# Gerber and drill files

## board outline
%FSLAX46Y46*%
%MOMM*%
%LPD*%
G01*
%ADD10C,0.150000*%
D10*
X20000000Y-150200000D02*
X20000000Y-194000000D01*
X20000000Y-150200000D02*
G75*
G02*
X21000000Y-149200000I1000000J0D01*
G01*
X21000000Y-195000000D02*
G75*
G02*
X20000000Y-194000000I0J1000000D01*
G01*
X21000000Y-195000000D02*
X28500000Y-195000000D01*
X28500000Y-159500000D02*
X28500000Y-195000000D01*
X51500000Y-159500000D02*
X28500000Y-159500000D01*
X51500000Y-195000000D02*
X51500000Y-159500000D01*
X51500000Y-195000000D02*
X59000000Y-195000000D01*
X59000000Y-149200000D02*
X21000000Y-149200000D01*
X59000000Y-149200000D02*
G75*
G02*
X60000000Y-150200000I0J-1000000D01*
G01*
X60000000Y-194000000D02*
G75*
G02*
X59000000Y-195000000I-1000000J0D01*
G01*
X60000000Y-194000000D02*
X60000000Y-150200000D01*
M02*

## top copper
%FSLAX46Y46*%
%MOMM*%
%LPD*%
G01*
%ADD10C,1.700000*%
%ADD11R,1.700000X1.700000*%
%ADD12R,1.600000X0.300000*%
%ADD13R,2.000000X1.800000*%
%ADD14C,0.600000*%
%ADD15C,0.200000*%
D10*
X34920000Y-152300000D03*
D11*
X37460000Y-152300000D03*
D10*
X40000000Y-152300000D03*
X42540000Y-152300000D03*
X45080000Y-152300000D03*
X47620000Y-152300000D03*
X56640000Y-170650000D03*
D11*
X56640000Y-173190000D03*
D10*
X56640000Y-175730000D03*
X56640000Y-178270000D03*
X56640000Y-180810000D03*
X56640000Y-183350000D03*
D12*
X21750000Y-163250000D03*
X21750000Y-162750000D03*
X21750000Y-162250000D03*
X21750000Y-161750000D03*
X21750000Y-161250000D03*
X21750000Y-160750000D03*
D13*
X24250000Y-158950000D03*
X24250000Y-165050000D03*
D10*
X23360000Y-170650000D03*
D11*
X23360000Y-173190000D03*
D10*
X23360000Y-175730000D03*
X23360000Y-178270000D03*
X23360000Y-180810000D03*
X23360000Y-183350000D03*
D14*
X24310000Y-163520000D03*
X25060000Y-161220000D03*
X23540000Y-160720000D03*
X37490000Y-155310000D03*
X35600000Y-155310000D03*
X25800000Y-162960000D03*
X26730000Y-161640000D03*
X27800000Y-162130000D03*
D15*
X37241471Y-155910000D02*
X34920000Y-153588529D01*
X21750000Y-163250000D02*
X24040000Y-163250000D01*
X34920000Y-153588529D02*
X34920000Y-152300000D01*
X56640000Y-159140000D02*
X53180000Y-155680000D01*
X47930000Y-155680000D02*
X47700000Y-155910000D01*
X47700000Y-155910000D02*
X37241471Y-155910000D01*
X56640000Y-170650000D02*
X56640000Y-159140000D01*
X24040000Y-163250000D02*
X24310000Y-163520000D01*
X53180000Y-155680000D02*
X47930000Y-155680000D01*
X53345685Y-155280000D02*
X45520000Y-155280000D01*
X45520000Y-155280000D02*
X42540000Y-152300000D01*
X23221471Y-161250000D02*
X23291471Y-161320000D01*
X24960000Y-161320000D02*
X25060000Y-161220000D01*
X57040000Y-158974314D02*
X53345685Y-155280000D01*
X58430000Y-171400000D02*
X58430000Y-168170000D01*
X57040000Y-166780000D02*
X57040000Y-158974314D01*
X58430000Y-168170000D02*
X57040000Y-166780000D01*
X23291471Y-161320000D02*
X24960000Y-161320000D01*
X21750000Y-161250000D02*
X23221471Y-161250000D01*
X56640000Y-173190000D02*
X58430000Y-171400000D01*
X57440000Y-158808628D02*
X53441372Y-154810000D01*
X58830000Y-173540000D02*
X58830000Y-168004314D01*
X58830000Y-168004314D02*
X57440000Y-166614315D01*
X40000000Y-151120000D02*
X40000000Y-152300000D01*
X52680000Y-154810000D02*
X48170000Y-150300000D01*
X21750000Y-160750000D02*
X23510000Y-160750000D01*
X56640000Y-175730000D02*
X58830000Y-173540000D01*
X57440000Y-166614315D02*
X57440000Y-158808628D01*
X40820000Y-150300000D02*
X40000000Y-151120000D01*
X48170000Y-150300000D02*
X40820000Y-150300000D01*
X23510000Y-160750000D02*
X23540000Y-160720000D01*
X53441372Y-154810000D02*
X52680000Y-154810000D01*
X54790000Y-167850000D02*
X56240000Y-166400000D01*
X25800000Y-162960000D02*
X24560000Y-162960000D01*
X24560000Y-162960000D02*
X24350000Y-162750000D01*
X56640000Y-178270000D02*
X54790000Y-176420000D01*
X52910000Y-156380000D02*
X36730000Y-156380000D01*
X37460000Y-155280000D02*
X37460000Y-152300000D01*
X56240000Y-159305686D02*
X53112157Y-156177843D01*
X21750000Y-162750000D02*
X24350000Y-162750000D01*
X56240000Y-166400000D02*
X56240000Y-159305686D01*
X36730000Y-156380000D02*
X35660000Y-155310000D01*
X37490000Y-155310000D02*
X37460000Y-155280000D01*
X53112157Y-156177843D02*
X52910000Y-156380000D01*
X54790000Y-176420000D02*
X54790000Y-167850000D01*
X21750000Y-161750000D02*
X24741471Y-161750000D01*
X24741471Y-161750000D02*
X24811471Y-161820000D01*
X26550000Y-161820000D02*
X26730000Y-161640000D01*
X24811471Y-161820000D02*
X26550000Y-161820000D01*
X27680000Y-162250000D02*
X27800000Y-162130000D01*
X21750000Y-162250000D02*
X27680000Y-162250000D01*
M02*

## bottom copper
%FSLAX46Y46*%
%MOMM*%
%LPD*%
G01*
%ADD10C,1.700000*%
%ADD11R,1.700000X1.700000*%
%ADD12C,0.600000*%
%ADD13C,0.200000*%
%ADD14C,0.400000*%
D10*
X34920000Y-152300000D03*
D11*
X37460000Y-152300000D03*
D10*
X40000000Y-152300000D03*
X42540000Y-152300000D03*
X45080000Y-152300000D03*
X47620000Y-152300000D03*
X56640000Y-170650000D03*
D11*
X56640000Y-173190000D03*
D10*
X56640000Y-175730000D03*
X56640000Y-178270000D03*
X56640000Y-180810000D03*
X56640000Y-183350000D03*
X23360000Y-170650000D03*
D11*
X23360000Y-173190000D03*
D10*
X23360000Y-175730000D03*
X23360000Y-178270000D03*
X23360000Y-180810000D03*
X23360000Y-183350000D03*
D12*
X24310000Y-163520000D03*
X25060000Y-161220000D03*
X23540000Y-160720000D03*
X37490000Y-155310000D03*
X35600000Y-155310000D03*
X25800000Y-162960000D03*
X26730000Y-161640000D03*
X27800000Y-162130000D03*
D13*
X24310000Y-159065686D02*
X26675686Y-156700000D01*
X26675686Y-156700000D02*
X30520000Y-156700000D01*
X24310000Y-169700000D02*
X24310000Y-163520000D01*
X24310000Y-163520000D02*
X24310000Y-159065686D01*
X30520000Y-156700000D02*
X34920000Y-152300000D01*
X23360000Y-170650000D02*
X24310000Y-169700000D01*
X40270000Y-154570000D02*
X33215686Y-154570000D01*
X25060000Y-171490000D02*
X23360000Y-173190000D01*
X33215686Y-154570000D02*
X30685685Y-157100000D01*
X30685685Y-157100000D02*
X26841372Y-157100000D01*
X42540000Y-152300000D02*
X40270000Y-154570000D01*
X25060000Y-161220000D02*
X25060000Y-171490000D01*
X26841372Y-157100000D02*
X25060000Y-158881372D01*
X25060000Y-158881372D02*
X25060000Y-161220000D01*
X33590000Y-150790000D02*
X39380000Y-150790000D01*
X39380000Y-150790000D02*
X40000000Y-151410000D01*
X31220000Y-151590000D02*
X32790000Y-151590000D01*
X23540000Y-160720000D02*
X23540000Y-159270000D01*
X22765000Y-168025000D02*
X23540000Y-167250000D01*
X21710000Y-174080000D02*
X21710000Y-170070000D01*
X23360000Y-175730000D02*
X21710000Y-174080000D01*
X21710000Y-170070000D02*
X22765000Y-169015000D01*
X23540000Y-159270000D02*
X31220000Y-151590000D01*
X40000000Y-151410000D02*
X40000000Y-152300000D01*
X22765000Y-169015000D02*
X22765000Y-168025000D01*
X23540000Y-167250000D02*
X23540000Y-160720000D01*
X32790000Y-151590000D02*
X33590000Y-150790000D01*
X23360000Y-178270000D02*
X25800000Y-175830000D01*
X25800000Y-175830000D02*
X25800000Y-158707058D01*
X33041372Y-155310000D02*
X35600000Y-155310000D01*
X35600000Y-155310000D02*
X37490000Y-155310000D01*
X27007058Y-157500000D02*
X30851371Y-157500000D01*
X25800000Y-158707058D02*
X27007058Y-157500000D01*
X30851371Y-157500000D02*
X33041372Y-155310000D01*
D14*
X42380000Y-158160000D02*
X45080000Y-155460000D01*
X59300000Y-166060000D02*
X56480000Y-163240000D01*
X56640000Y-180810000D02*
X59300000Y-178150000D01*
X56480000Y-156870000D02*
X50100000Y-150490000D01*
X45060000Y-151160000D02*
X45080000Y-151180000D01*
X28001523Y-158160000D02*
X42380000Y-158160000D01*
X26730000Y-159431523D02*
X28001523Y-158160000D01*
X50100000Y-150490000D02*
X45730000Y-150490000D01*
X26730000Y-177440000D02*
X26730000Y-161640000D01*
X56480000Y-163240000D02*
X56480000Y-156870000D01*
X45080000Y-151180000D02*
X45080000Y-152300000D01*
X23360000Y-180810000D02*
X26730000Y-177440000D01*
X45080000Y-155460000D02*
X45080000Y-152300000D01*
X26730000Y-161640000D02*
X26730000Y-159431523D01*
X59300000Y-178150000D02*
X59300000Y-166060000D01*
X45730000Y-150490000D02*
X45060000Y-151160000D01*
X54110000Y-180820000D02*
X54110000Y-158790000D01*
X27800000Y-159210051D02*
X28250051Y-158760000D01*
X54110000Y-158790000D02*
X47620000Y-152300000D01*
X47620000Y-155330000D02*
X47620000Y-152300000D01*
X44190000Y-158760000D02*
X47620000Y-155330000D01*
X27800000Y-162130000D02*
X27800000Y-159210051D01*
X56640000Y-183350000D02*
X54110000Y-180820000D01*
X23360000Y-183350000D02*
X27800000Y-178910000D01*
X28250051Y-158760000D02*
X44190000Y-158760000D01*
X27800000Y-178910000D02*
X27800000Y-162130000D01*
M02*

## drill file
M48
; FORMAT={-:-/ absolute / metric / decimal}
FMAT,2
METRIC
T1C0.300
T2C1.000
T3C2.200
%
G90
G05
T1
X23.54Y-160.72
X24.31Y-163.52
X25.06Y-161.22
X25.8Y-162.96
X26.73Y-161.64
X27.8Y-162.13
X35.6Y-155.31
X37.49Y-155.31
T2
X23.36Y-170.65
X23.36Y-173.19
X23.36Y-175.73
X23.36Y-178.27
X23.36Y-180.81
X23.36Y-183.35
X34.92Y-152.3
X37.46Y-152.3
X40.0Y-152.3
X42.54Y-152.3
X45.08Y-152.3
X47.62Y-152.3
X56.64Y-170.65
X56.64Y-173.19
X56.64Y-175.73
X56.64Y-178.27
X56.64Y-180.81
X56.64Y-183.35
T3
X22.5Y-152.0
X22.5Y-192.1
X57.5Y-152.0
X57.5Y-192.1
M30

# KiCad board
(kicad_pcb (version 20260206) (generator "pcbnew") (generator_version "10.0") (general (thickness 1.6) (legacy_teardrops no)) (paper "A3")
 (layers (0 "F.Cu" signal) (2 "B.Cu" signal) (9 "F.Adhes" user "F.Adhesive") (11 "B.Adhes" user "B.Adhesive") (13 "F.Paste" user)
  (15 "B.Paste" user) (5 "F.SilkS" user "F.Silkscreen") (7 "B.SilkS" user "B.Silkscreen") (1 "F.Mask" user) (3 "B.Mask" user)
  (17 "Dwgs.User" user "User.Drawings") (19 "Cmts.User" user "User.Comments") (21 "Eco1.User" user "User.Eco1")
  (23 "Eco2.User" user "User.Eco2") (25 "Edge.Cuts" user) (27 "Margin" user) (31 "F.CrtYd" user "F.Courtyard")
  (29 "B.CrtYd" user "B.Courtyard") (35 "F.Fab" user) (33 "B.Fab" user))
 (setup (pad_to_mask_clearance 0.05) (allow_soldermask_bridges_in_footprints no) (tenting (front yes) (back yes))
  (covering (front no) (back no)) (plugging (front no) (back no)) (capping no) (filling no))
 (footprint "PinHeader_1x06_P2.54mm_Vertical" (layer "F.Cu") (at 41.27 152.3 90)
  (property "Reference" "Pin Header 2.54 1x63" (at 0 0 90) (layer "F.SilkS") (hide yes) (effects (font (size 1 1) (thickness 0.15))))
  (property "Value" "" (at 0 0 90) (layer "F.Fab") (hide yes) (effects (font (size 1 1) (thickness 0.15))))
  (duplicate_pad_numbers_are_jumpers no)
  (pad "1" thru_hole circle (at 0 -6.35 90) (size 1.7 1.7) (drill 1) (layers "*.Cu" "*.Mask") (remove_unused_layers no) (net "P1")
   (thermal_bridge_angle 90))
  (pad "2" thru_hole rect (at 0 -3.81 90) (size 1.7 1.7) (drill 1) (layers "*.Cu" "*.Mask") (remove_unused_layers no) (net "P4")
   (thermal_bridge_angle 45))
  (pad "3" thru_hole circle (at 0 -1.27 90) (size 1.7 1.7) (drill 1) (layers "*.Cu" "*.Mask") (remove_unused_layers no) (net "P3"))
  (pad "4" thru_hole circle (at 0 1.27 90) (size 1.7 1.7) (drill 1) (layers "*.Cu" "*.Mask") (remove_unused_layers no) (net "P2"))
  (pad "5" thru_hole circle (at 0 3.81 90) (size 1.7 1.7) (drill 1) (layers "*.Cu" "*.Mask") (remove_unused_layers no) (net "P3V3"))
  (pad "6" thru_hole circle (at 0 6.35 90) (size 1.7 1.7) (drill 1) (layers "*.Cu" "*.Mask") (remove_unused_layers no) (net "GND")))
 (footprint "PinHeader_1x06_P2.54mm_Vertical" (layer "F.Cu") (at 56.64 177)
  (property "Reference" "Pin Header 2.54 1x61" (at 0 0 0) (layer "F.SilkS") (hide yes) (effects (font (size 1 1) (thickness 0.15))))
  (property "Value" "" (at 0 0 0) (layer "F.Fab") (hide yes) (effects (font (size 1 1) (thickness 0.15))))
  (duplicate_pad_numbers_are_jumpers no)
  (pad "1" thru_hole circle (at 0 -6.35) (size 1.7 1.7) (drill 1) (layers "*.Cu" "*.Mask") (remove_unused_layers no) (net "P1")
   (thermal_bridge_angle 90))
  (pad "2" thru_hole rect (at 0 -3.81) (size 1.7 1.7) (drill 1) (layers "*.Cu" "*.Mask") (remove_unused_layers no) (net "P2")
   (thermal_bridge_angle 45))
  (pad "3" thru_hole circle (at 0 -1.27) (size 1.7 1.7) (drill 1) (layers "*.Cu" "*.Mask") (remove_unused_layers no) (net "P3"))
  (pad "4" thru_hole circle (at 0 1.27) (size 1.7 1.7) (drill 1) (layers "*.Cu" "*.Mask") (remove_unused_layers no) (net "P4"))
  (pad "5" thru_hole circle (at 0 3.81) (size 1.7 1.7) (drill 1) (layers "*.Cu" "*.Mask") (remove_unused_layers no) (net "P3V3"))
  (pad "6" thru_hole circle (at 0 6.35) (size 1.7 1.7) (drill 1) (layers "*.Cu" "*.Mask") (remove_unused_layers no) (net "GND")))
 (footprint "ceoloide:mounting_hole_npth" (layer "F.Cu") (at 57.5 152)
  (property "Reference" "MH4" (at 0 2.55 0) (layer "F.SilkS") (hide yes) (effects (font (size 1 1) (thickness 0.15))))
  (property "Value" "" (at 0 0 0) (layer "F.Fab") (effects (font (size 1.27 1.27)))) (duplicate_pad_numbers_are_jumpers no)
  (pad "" np_thru_hole circle (at 0 0) (size 2.2 2.2) (drill 2.2) (layers "*.Cu" "*.Mask")))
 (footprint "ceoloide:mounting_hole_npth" (layer "F.Cu") (at 22.5 192.1)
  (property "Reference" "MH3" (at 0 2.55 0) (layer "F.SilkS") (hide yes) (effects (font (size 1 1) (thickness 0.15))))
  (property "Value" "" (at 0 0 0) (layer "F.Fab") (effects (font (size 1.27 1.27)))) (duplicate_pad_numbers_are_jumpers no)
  (pad "" np_thru_hole circle (at 0 0) (size 2.2 2.2) (drill 2.2) (layers "*.Cu" "*.Mask")))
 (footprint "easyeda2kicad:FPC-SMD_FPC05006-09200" (layer "F.Cu") (at 23 162 90)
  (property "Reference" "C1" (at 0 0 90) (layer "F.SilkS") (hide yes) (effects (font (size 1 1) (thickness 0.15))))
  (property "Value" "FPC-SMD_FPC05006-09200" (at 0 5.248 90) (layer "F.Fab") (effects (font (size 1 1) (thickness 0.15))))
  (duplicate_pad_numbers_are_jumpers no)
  (pad "1" smd rect (at -1.25 -1.25 90) (size 0.3 1.6) (layers "F.Cu" "F.Mask" "F.Paste") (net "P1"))
  (pad "2" smd rect (at -0.75 -1.25 90) (size 0.3 1.6) (layers "F.Cu" "F.Mask" "F.Paste") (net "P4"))
  (pad "3" smd rect (at -0.25 -1.25 90) (size 0.3 1.6) (layers "F.Cu" "F.Mask" "F.Paste") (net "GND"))
  (pad "4" smd rect (at 0.25 -1.25 90) (size 0.3 1.6) (layers "F.Cu" "F.Mask" "F.Paste") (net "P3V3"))
  (pad "5" smd rect (at 0.75 -1.25 90) (size 0.3 1.6) (layers "F.Cu" "F.Mask" "F.Paste") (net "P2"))
  (pad "6" smd rect (at 1.25 -1.25 90) (size 0.3 1.6) (layers "F.Cu" "F.Mask" "F.Paste") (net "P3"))
  (pad "7" smd rect (at 3.05 1.25 90) (size 1.8 2) (layers "F.Cu" "F.Mask" "F.Paste"))
  (pad "8" smd rect (at -3.05 1.25 90) (size 1.8 2) (layers "F.Cu" "F.Mask" "F.Paste")))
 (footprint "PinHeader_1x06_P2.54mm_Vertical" (layer "F.Cu") (at 23.36 177)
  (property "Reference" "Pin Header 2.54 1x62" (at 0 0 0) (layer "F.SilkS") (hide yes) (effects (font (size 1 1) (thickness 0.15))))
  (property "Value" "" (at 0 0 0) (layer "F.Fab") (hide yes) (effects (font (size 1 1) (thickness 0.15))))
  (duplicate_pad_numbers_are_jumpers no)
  (pad "1" thru_hole circle (at 0 -6.35) (size 1.7 1.7) (drill 1) (layers "*.Cu" "*.Mask") (remove_unused_layers no) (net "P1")
   (thermal_bridge_angle 90))
  (pad "2" thru_hole rect (at 0 -3.81) (size 1.7 1.7) (drill 1) (layers "*.Cu" "*.Mask") (remove_unused_layers no) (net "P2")
   (thermal_bridge_angle 45))
  (pad "3" thru_hole circle (at 0 -1.27) (size 1.7 1.7) (drill 1) (layers "*.Cu" "*.Mask") (remove_unused_layers no) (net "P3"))
  (pad "4" thru_hole circle (at 0 1.27) (size 1.7 1.7) (drill 1) (layers "*.Cu" "*.Mask") (remove_unused_layers no) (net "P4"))
  (pad "5" thru_hole circle (at 0 3.81) (size 1.7 1.7) (drill 1) (layers "*.Cu" "*.Mask") (remove_unused_layers no) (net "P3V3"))
  (pad "6" thru_hole circle (at 0 6.35) (size 1.7 1.7) (drill 1) (layers "*.Cu" "*.Mask") (remove_unused_layers no) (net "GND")))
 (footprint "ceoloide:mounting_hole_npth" (layer "F.Cu") (at 57.5 192.1)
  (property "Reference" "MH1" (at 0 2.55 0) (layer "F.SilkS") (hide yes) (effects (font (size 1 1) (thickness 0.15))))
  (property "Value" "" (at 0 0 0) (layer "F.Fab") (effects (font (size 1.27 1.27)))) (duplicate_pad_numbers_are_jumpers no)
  (pad "" np_thru_hole circle (at 0 0) (size 2.2 2.2) (drill 2.2) (layers "*.Cu" "*.Mask")))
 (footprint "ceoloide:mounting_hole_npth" (layer "F.Cu") (at 22.5 152)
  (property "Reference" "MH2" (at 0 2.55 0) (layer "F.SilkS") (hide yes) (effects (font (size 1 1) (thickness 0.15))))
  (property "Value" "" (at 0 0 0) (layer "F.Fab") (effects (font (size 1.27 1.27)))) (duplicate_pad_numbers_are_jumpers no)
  (pad "" np_thru_hole circle (at 0 0) (size 2.2 2.2) (drill 2.2) (layers "*.Cu" "*.Mask")))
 (gr_line (start 20 150.2) (end 20 194) (stroke (width 0.15) (type default)) (layer "Edge.Cuts"))
 (gr_arc (start 20 150.2) (mid 20.292893 149.492893) (end 21 149.2) (stroke (width 0.15) (type default)) (layer "Edge.Cuts"))
 (gr_arc (start 21 195) (mid 20.292893 194.707107) (end 20 194) (stroke (width 0.15) (type default)) (layer "Edge.Cuts"))
 (gr_line (start 21 195) (end 28.5 195) (stroke (width 0.15) (type default)) (layer "Edge.Cuts"))
 (gr_line (start 28.5 159.5) (end 28.5 195) (stroke (width 0.15) (type default)) (layer "Edge.Cuts"))
 (gr_line (start 51.5 159.5) (end 28.5 159.5) (stroke (width 0.15) (type default)) (layer "Edge.Cuts"))
 (gr_line (start 51.5 195) (end 51.5 159.5) (stroke (width 0.15) (type default)) (layer "Edge.Cuts"))
 (gr_line (start 51.5 195) (end 59 195) (stroke (width 0.15) (type default)) (layer "Edge.Cuts"))
 (gr_line (start 59 149.2) (end 21 149.2) (stroke (width 0.15) (type default)) (layer "Edge.Cuts"))
 (gr_arc (start 59 149.2) (mid 59.707107 149.492893) (end 60 150.2) (stroke (width 0.15) (type default)) (layer "Edge.Cuts"))
 (gr_arc (start 60 194) (mid 59.707107 194.707107) (end 59 195) (stroke (width 0.15) (type default)) (layer "Edge.Cuts"))
 (gr_line (start 60 194) (end 60 150.2) (stroke (width 0.15) (type default)) (layer "Edge.Cuts"))
 (segment (start 37.241471 155.91) (end 34.92 153.588529) (width 0.2) (layer "F.Cu") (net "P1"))
 (segment (start 21.75 163.25) (end 24.04 163.25) (width 0.2) (layer "F.Cu") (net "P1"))
 (segment (start 34.92 153.588529) (end 34.92 152.3) (width 0.2) (layer "F.Cu") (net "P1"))
 (segment (start 56.64 159.14) (end 53.18 155.68) (width 0.2) (layer "F.Cu") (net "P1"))
 (segment (start 47.93 155.68) (end 47.7 155.91) (width 0.2) (layer "F.Cu") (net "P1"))
 (segment (start 47.7 155.91) (end 37.241471 155.91) (width 0.2) (layer "F.Cu") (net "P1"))
 (segment (start 56.64 170.65) (end 56.64 159.14) (width 0.2) (layer "F.Cu") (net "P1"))
 (segment (start 24.04 163.25) (end 24.31 163.52) (width 0.2) (layer "F.Cu") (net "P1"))
 (segment (start 53.18 155.68) (end 47.93 155.68) (width 0.2) (layer "F.Cu") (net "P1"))
 (via (at 24.31 163.52) (size 0.6) (drill 0.3) (layers "F.Cu" "B.Cu") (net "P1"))
 (segment (start 24.31 159.065686) (end 26.675686 156.7) (width 0.2) (layer "B.Cu") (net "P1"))
 (segment (start 26.675686 156.7) (end 30.52 156.7) (width 0.2) (layer "B.Cu") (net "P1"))
 (segment (start 24.31 169.7) (end 24.31 163.52) (width 0.2) (layer "B.Cu") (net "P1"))
 (segment (start 24.31 163.52) (end 24.31 159.065686) (width 0.2) (layer "B.Cu") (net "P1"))
 (segment (start 30.52 156.7) (end 34.92 152.3) (width 0.2) (layer "B.Cu") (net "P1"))
 (segment (start 23.36 170.65) (end 24.31 169.7) (width 0.2) (layer "B.Cu") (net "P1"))
 (segment (start 53.345685 155.28) (end 45.52 155.28) (width 0.2) (layer "F.Cu") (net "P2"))
 (segment (start 45.52 155.28) (end 42.54 152.3) (width 0.2) (layer "F.Cu") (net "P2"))
 (segment (start 23.221471 161.25) (end 23.291471 161.32) (width 0.2) (layer "F.Cu") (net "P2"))
 (segment (start 24.96 161.32) (end 25.06 161.22) (width 0.2) (layer "F.Cu") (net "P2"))
 (segment (start 57.04 158.974314) (end 53.345685 155.28) (width 0.2) (layer "F.Cu") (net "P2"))
 (segment (start 58.43 171.4) (end 58.43 168.17) (width 0.2) (layer "F.Cu") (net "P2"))
 (segment (start 57.04 166.78) (end 57.04 158.974314) (width 0.2) (layer "F.Cu") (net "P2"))
 (segment (start 58.43 168.17) (end 57.04 166.78) (width 0.2) (layer "F.Cu") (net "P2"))
 (segment (start 23.291471 161.32) (end 24.96 161.32) (width 0.2) (layer "F.Cu") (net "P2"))
 (segment (start 21.75 161.25) (end 23.221471 161.25) (width 0.2) (layer "F.Cu") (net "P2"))
 (segment (start 56.64 173.19) (end 58.43 171.4) (width 0.2) (layer "F.Cu") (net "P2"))
 (via (at 25.06 161.22) (size 0.6) (drill 0.3) (layers "F.Cu" "B.Cu") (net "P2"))
 (segment (start 40.27 154.57) (end 33.215686 154.57) (width 0.2) (layer "B.Cu") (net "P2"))
 (segment (start 25.06 171.49) (end 23.36 173.19) (width 0.2) (layer "B.Cu") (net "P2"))
 (segment (start 33.215686 154.57) (end 30.685685 157.1) (width 0.2) (layer "B.Cu") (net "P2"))
 (segment (start 30.685685 157.1) (end 26.841372 157.1) (width 0.2) (layer "B.Cu") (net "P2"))
 (segment (start 42.54 152.3) (end 40.27 154.57) (width 0.2) (layer "B.Cu") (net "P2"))
 (segment (start 25.06 161.22) (end 25.06 171.49) (width 0.2) (layer "B.Cu") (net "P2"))
 (segment (start 26.841372 157.1) (end 25.06 158.881372) (width 0.2) (layer "B.Cu") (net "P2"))
 (segment (start 25.06 158.881372) (end 25.06 161.22) (width 0.2) (layer "B.Cu") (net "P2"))
 (segment (start 57.44 158.808628) (end 53.441372 154.81) (width 0.2) (layer "F.Cu") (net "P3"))
 (segment (start 58.83 173.54) (end 58.83 168.004314) (width 0.2) (layer "F.Cu") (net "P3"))
 (segment (start 58.83 168.004314) (end 57.44 166.614315) (width 0.2) (layer "F.Cu") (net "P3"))
 (segment (start 40 151.12) (end 40 152.3) (width 0.2) (layer "F.Cu") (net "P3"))
 (segment (start 52.68 154.81) (end 48.17 150.3) (width 0.2) (layer "F.Cu") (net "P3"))
 (segment (start 21.75 160.75) (end 23.51 160.75) (width 0.2) (layer "F.Cu") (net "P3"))
 (segment (start 56.64 175.73) (end 58.83 173.54) (width 0.2) (layer "F.Cu") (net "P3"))
 (segment (start 57.44 166.614315) (end 57.44 158.808628) (width 0.2) (layer "F.Cu") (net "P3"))
 (segment (start 40.82 150.3) (end 40 151.12) (width 0.2) (layer "F.Cu") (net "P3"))
 (segment (start 48.17 150.3) (end 40.82 150.3) (width 0.2) (layer "F.Cu") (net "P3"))
 (segment (start 23.51 160.75) (end 23.54 160.72) (width 0.2) (layer "F.Cu") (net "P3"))
 (segment (start 53.441372 154.81) (end 52.68 154.81) (width 0.2) (layer "F.Cu") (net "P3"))
 (via (at 23.54 160.72) (size 0.6) (drill 0.3) (layers "F.Cu" "B.Cu") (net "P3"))
 (segment (start 33.59 150.79) (end 39.38 150.79) (width 0.2) (layer "B.Cu") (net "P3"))
 (segment (start 39.38 150.79) (end 40 151.41) (width 0.2) (layer "B.Cu") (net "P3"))
 (segment (start 31.22 151.59) (end 32.79 151.59) (width 0.2) (layer "B.Cu") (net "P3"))
 (segment (start 23.54 160.72) (end 23.54 159.27) (width 0.2) (layer "B.Cu") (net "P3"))
 (segment (start 22.765 168.025) (end 23.54 167.25) (width 0.2) (layer "B.Cu") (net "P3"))
 (segment (start 21.71 174.08) (end 21.71 170.07) (width 0.2) (layer "B.Cu") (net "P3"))
 (segment (start 23.36 175.73) (end 21.71 174.08) (width 0.2) (layer "B.Cu") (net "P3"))
 (segment (start 21.71 170.07) (end 22.765 169.015) (width 0.2) (layer "B.Cu") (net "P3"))
 (segment (start 23.54 159.27) (end 31.22 151.59) (width 0.2) (layer "B.Cu") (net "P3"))
 (segment (start 40 151.41) (end 40 152.3) (width 0.2) (layer "B.Cu") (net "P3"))
 (segment (start 22.765 169.015) (end 22.765 168.025) (width 0.2) (layer "B.Cu") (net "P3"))
 (segment (start 23.54 167.25) (end 23.54 160.72) (width 0.2) (layer "B.Cu") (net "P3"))
 (segment (start 32.79 151.59) (end 33.59 150.79) (width 0.2) (layer "B.Cu") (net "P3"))
 (segment (start 54.79 167.85) (end 56.24 166.4) (width 0.2) (layer "F.Cu") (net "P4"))
 (segment (start 25.8 162.96) (end 24.56 162.96) (width 0.2) (layer "F.Cu") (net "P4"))
 (segment (start 24.56 162.96) (end 24.35 162.75) (width 0.2) (layer "F.Cu") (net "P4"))
 (segment (start 56.64 178.27) (end 54.79 176.42) (width 0.2) (layer "F.Cu") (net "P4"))
 (segment (start 52.91 156.38) (end 36.73 156.38) (width 0.2) (layer "F.Cu") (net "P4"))
 (segment (start 37.46 155.28) (end 37.46 152.3) (width 0.2) (layer "F.Cu") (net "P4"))
 (segment (start 56.24 159.305686) (end 53.112157 156.177843) (width 0.2) (layer "F.Cu") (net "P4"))
 (segment (start 21.75 162.75) (end 24.35 162.75) (width 0.2) (layer "F.Cu") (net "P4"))
 (segment (start 56.24 166.4) (end 56.24 159.305686) (width 0.2) (layer "F.Cu") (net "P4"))
 (segment (start 36.73 156.38) (end 35.66 155.31) (width 0.2) (layer "F.Cu") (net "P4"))
 (segment (start 37.49 155.31) (end 37.46 155.28) (width 0.2) (layer "F.Cu") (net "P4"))
 (segment (start 53.112157 156.177843) (end 52.91 156.38) (width 0.2) (layer "F.Cu") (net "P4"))
 (segment (start 54.79 176.42) (end 54.79 167.85) (width 0.2) (layer "F.Cu") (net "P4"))
 (via (at 37.49 155.31) (size 0.6) (drill 0.3) (layers "F.Cu" "B.Cu") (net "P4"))
 (via (at 35.6 155.31) (size 0.6) (drill 0.3) (layers "F.Cu" "B.Cu") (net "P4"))
 (via (at 25.8 162.96) (size 0.6) (drill 0.3) (layers "F.Cu" "B.Cu") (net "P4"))
 (segment (start 23.36 178.27) (end 25.8 175.83) (width 0.2) (layer "B.Cu") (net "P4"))
 (segment (start 25.8 175.83) (end 25.8 158.707058) (width 0.2) (layer "B.Cu") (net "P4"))
 (segment (start 33.041372 155.31) (end 35.6 155.31) (width 0.2) (layer "B.Cu") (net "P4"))
 (segment (start 35.6 155.31) (end 37.49 155.31) (width 0.2) (layer "B.Cu") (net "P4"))
 (segment (start 27.007058 157.5) (end 30.851371 157.5) (width 0.2) (layer "B.Cu") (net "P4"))
 (segment (start 25.8 158.707058) (end 27.007058 157.5) (width 0.2) (layer "B.Cu") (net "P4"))
 (segment (start 30.851371 157.5) (end 33.041372 155.31) (width 0.2) (layer "B.Cu") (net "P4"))
 (segment (start 21.75 161.75) (end 24.741471 161.75) (width 0.2) (layer "F.Cu") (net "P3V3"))
 (segment (start 24.741471 161.75) (end 24.811471 161.82) (width 0.2) (layer "F.Cu") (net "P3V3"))
 (segment (start 26.55 161.82) (end 26.73 161.64) (width 0.2) (layer "F.Cu") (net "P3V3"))
 (segment (start 24.811471 161.82) (end 26.55 161.82) (width 0.2) (layer "F.Cu") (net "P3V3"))
 (via (at 26.73 161.64) (size 0.6) (drill 0.3) (layers "F.Cu" "B.Cu") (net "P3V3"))
 (segment (start 42.38 158.16) (end 45.08 155.46) (width 0.4) (layer "B.Cu") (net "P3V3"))
 (segment (start 59.3 166.06) (end 56.48 163.24) (width 0.4) (layer "B.Cu") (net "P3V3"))
 (segment (start 56.64 180.81) (end 59.3 178.15) (width 0.4) (layer "B.Cu") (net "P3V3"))
 (segment (start 56.48 156.87) (end 50.1 150.49) (width 0.4) (layer "B.Cu") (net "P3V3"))
 (segment (start 45.06 151.16) (end 45.08 151.18) (width 0.4) (layer "B.Cu") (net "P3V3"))
 (segment (start 28.001523 158.16) (end 42.38 158.16) (width 0.4) (layer "B.Cu") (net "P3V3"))
 (segment (start 26.73 159.431523) (end 28.001523 158.16) (width 0.4) (layer "B.Cu") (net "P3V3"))
 (segment (start 50.1 150.49) (end 45.73 150.49) (width 0.4) (layer "B.Cu") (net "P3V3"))
 (segment (start 26.73 177.44) (end 26.73 161.64) (width 0.4) (layer "B.Cu") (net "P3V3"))
 (segment (start 56.48 163.24) (end 56.48 156.87) (width 0.4) (layer "B.Cu") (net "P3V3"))
 (segment (start 45.08 151.18) (end 45.08 152.3) (width 0.4) (layer "B.Cu") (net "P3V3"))
 (segment (start 23.36 180.81) (end 26.73 177.44) (width 0.4) (layer "B.Cu") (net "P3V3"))
 (segment (start 45.08 155.46) (end 45.08 152.3) (width 0.4) (layer "B.Cu") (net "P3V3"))
 (segment (start 26.73 161.64) (end 26.73 159.431523) (width 0.4) (layer "B.Cu") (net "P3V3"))
 (segment (start 59.3 178.15) (end 59.3 166.06) (width 0.4) (layer "B.Cu") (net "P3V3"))
 (segment (start 45.73 150.49) (end 45.06 151.16) (width 0.4) (layer "B.Cu") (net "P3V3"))
 (segment (start 27.68 162.25) (end 27.8 162.13) (width 0.2) (layer "F.Cu") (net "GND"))
 (segment (start 21.75 162.25) (end 27.68 162.25) (width 0.2) (layer "F.Cu") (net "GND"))
 (via (at 27.8 162.13) (size 0.6) (drill 0.3) (layers "F.Cu" "B.Cu") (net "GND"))
 (segment (start 54.11 180.82) (end 54.11 158.79) (width 0.4) (layer "B.Cu") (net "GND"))
 (segment (start 27.8 159.210051) (end 28.250051 158.76) (width 0.4) (layer "B.Cu") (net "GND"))
 (segment (start 54.11 158.79) (end 47.62 152.3) (width 0.4) (layer "B.Cu") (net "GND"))
 (segment (start 47.62 155.33) (end 47.62 152.3) (width 0.4) (layer "B.Cu") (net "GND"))
 (segment (start 44.19 158.76) (end 47.62 155.33) (width 0.4) (layer "B.Cu") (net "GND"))
 (segment (start 27.8 162.13) (end 27.8 159.210051) (width 0.4) (layer "B.Cu") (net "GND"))
 (segment (start 56.64 183.35) (end 54.11 180.82) (width 0.4) (layer "B.Cu") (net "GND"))
 (segment (start 23.36 183.35) (end 27.8 178.91) (width 0.4) (layer "B.Cu") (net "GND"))
 (segment (start 28.250051 158.76) (end 44.19 158.76) (width 0.4) (layer "B.Cu") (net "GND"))
 (segment (start 27.8 178.91) (end 27.8 162.13) (width 0.4) (layer "B.Cu") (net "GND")))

